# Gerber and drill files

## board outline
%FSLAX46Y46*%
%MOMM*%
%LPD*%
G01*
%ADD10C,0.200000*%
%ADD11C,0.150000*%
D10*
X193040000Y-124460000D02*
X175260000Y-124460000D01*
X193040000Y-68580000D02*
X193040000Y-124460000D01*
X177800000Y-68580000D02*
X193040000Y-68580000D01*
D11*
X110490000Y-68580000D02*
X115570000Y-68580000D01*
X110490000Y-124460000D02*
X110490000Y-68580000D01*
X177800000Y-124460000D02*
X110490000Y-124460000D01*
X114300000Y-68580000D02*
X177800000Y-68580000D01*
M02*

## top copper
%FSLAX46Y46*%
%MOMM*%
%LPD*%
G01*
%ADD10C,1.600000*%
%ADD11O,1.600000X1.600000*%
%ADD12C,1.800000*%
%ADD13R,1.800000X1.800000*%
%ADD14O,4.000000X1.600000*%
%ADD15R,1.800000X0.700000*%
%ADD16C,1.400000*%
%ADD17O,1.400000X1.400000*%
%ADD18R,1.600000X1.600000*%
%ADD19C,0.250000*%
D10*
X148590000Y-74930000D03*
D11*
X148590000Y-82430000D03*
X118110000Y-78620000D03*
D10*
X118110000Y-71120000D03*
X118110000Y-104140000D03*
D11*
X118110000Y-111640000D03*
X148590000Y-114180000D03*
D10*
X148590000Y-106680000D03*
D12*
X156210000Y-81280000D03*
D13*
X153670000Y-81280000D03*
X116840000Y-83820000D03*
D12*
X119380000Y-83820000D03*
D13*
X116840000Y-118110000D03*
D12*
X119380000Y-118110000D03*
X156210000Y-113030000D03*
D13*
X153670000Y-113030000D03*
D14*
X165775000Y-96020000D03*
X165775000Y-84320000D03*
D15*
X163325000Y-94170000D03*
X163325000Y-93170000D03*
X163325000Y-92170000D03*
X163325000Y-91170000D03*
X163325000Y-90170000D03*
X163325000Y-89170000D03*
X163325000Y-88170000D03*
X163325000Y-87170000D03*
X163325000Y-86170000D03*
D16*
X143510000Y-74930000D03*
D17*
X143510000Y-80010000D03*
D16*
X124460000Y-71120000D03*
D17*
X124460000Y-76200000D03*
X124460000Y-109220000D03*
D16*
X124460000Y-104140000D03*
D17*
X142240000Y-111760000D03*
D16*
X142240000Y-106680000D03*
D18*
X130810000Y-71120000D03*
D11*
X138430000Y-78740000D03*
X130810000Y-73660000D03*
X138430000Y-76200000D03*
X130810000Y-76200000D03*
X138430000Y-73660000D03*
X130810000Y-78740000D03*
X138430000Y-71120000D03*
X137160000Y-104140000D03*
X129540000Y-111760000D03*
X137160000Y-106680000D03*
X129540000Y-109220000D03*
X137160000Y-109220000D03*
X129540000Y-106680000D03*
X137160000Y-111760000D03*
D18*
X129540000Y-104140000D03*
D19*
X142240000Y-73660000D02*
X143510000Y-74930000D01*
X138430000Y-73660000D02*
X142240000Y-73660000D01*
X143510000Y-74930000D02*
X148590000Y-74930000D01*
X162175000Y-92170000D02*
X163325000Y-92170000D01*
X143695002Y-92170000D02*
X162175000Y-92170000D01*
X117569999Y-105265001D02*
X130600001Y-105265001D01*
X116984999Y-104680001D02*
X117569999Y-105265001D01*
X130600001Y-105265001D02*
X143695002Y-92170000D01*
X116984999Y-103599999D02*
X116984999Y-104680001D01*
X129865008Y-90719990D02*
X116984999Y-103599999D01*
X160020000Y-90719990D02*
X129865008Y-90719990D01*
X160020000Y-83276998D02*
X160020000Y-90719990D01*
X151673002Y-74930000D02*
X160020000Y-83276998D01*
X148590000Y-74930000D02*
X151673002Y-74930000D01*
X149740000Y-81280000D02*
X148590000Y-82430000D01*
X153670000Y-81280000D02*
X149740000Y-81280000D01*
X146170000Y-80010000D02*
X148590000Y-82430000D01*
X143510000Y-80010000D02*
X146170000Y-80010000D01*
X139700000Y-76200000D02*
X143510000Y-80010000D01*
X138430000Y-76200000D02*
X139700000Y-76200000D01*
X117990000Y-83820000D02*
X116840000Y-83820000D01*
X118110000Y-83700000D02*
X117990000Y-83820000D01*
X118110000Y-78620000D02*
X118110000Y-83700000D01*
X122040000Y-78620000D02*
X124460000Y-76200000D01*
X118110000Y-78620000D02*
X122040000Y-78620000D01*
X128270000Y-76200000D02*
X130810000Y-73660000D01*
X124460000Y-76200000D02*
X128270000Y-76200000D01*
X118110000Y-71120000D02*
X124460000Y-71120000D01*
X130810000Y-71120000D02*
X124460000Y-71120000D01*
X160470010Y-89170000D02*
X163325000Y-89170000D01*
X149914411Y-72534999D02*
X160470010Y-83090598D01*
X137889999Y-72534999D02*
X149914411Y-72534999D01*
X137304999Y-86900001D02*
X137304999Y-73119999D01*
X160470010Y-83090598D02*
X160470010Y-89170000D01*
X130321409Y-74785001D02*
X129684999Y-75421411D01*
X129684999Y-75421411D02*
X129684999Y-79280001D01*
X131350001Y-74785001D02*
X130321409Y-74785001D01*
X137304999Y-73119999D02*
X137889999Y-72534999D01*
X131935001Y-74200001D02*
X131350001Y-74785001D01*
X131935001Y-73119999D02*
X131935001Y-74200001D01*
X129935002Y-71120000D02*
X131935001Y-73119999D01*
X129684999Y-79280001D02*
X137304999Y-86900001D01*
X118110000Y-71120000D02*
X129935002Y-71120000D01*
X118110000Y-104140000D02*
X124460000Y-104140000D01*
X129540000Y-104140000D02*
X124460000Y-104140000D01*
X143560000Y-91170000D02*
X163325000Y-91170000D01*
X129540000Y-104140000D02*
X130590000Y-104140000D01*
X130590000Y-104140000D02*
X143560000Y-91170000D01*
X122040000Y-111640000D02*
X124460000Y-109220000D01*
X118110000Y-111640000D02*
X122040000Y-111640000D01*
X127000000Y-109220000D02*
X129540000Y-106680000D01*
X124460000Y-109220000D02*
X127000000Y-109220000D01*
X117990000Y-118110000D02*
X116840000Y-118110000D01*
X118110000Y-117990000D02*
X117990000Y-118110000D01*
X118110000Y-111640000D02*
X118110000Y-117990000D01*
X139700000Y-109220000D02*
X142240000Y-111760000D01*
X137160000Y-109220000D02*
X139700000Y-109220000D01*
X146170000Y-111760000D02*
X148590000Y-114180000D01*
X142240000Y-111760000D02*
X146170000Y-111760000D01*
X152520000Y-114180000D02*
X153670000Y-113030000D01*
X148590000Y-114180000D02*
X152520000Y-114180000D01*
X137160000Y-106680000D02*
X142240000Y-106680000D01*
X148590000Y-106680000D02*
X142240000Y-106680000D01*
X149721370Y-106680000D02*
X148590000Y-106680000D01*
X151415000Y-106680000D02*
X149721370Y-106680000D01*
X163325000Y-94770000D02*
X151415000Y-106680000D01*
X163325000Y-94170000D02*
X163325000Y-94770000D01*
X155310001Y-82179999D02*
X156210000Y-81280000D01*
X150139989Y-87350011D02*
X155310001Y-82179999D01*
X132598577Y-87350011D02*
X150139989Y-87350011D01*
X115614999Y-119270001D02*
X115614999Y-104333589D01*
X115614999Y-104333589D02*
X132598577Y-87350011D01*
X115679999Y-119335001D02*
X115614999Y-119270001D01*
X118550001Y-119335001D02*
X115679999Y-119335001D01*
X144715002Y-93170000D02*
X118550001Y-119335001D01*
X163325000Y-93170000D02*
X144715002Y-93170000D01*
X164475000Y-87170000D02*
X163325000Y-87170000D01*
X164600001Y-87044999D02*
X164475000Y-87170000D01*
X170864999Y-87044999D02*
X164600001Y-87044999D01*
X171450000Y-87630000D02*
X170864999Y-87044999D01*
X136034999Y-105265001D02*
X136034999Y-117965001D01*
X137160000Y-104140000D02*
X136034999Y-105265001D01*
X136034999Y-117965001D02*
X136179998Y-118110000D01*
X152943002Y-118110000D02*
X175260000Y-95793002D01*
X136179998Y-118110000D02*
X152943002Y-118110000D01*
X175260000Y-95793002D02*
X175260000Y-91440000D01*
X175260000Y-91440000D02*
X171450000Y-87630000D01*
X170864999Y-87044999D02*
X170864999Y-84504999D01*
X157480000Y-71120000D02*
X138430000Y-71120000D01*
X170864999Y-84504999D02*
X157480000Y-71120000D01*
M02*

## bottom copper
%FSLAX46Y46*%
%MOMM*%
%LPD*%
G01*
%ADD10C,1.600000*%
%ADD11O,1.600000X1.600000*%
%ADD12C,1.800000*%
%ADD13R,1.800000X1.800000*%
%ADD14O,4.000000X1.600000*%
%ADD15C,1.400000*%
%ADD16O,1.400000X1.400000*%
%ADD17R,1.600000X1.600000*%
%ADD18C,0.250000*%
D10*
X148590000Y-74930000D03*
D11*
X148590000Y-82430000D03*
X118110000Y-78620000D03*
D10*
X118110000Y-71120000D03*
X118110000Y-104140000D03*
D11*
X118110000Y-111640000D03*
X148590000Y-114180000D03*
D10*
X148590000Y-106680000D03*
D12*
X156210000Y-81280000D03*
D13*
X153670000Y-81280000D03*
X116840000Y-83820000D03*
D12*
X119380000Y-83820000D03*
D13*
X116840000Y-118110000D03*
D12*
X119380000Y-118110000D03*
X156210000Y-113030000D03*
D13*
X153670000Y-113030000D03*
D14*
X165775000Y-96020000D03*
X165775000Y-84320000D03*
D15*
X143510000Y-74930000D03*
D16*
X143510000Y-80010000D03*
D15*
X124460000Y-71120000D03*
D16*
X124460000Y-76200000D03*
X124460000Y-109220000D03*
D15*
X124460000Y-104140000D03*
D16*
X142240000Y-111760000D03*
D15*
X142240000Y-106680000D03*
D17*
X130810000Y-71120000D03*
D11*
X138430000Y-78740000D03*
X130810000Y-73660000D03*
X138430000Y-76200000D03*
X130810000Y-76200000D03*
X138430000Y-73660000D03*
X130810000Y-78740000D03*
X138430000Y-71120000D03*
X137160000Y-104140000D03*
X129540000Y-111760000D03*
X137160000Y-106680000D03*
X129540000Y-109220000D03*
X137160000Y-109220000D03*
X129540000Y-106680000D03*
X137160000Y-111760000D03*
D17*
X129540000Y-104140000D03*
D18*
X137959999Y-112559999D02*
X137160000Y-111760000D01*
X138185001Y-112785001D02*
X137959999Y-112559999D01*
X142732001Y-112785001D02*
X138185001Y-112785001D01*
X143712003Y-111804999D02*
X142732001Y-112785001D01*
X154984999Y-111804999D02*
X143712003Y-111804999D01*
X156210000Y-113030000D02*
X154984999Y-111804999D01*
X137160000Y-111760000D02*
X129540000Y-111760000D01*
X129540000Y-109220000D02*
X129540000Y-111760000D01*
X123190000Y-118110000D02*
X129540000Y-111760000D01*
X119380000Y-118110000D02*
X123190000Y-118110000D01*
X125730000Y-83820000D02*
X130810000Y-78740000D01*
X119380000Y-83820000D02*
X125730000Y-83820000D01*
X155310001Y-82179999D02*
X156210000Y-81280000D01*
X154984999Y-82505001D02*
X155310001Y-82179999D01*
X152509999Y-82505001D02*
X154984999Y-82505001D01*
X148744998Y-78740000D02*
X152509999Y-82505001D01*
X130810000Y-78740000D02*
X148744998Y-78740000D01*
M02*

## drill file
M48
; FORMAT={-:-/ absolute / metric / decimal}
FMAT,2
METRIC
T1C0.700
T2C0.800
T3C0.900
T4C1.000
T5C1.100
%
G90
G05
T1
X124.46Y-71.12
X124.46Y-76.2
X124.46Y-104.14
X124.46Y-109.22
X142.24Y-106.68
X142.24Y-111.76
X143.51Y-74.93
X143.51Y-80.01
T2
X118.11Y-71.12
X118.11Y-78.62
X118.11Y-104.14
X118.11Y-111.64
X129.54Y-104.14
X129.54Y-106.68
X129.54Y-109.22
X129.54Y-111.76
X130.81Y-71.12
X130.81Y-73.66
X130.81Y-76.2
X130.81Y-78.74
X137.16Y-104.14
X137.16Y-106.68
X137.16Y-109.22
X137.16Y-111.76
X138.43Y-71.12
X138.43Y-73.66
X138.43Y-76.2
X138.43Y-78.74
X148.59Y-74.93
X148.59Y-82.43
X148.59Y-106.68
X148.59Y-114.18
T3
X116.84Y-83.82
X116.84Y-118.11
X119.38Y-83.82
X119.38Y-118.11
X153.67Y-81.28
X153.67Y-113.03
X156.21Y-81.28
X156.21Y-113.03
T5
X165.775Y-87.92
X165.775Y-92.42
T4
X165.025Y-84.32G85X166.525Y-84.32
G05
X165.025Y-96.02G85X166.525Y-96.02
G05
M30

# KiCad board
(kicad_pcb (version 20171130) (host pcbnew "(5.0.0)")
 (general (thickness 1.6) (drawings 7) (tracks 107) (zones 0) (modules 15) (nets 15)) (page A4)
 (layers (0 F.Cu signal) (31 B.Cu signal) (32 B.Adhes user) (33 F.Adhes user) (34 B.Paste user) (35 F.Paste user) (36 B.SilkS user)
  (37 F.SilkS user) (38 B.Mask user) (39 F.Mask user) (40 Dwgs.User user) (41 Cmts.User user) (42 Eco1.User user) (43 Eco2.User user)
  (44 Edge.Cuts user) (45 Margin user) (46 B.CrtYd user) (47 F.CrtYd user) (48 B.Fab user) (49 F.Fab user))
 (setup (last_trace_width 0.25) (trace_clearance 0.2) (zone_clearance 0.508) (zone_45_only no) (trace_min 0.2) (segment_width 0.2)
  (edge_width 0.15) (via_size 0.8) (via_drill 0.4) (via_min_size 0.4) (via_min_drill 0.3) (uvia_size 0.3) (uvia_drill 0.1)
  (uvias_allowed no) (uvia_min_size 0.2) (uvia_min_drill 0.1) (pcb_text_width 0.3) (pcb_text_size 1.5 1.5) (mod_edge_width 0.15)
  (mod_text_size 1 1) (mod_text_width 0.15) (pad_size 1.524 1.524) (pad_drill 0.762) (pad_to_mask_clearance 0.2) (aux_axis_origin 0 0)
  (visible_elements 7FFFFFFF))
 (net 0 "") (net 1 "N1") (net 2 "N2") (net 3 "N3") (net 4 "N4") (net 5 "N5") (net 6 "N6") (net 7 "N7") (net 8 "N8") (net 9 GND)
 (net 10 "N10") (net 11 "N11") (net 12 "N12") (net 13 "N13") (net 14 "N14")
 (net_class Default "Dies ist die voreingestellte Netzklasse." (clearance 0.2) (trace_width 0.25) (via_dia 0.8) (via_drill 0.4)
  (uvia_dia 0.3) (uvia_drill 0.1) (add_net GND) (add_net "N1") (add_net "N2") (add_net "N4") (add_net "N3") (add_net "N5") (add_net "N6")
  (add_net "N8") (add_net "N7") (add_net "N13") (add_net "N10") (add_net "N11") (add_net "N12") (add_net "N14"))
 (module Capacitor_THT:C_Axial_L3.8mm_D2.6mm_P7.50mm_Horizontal (layer F.Cu) (at 148.59 74.93 270)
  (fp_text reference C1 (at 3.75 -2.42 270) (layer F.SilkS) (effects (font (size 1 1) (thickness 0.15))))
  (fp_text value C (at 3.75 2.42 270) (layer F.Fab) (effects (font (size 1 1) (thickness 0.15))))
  (pad 1 thru_hole circle (at 0 0 270) (size 1.6 1.6) (drill 0.8) (layers *.Cu *.Mask) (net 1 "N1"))
  (pad 2 thru_hole oval (at 7.5 0 270) (size 1.6 1.6) (drill 0.8) (layers *.Cu *.Mask) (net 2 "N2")))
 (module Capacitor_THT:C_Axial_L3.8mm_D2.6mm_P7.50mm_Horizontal (layer F.Cu) (at 118.11 71.12 270)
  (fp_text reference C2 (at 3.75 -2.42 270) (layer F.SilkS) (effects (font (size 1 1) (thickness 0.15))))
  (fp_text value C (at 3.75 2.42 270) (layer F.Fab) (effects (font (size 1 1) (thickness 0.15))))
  (pad 2 thru_hole oval (at 7.5 0 270) (size 1.6 1.6) (drill 0.8) (layers *.Cu *.Mask) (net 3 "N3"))
  (pad 1 thru_hole circle (at 0 0 270) (size 1.6 1.6) (drill 0.8) (layers *.Cu *.Mask) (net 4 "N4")))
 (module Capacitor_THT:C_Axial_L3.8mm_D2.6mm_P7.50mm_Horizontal (layer F.Cu) (at 118.11 104.14 270)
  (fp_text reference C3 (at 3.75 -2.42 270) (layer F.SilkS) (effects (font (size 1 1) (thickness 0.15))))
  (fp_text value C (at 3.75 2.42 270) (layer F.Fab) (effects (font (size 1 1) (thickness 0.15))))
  (pad 1 thru_hole circle (at 0 0 270) (size 1.6 1.6) (drill 0.8) (layers *.Cu *.Mask) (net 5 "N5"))
  (pad 2 thru_hole oval (at 7.5 0 270) (size 1.6 1.6) (drill 0.8) (layers *.Cu *.Mask) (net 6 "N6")))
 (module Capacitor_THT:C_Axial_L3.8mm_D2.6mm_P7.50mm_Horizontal (layer F.Cu) (at 148.59 106.68 270)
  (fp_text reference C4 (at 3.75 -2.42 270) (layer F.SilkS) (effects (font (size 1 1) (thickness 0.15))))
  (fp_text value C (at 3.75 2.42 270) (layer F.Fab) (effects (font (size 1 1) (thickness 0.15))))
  (pad 2 thru_hole oval (at 7.5 0 270) (size 1.6 1.6) (drill 0.8) (layers *.Cu *.Mask) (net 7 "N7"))
  (pad 1 thru_hole circle (at 0 0 270) (size 1.6 1.6) (drill 0.8) (layers *.Cu *.Mask) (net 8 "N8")))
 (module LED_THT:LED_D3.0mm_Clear (layer F.Cu) (at 153.67 81.28)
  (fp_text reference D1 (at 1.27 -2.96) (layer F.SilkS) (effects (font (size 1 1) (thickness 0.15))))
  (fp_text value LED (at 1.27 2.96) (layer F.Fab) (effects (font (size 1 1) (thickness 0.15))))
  (pad 2 thru_hole circle (at 2.54 0) (size 1.8 1.8) (drill 0.9) (layers *.Cu *.Mask) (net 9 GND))
  (pad 1 thru_hole rect (at 0 0) (size 1.8 1.8) (drill 0.9) (layers *.Cu *.Mask) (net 2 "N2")))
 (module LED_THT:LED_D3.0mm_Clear (layer F.Cu) (at 116.84 83.82)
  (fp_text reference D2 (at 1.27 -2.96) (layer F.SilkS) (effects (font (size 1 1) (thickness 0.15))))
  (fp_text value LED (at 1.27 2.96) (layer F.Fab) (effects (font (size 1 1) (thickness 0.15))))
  (pad 1 thru_hole rect (at 0 0) (size 1.8 1.8) (drill 0.9) (layers *.Cu *.Mask) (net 3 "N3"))
  (pad 2 thru_hole circle (at 2.54 0) (size 1.8 1.8) (drill 0.9) (layers *.Cu *.Mask) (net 9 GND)))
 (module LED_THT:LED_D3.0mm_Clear (layer F.Cu) (at 116.84 118.11)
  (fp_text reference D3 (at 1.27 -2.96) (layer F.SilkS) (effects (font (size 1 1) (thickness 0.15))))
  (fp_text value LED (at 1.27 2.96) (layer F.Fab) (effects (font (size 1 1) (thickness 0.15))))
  (pad 1 thru_hole rect (at 0 0) (size 1.8 1.8) (drill 0.9) (layers *.Cu *.Mask) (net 6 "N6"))
  (pad 2 thru_hole circle (at 2.54 0) (size 1.8 1.8) (drill 0.9) (layers *.Cu *.Mask) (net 9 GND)))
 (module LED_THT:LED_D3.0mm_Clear (layer F.Cu) (at 153.67 113.03)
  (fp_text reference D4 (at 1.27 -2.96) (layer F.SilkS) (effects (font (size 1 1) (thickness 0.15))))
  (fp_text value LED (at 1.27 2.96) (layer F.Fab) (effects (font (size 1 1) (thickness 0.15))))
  (pad 2 thru_hole circle (at 2.54 0) (size 1.8 1.8) (drill 0.9) (layers *.Cu *.Mask) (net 9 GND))
  (pad 1 thru_hole rect (at 0 0) (size 1.8 1.8) (drill 0.9) (layers *.Cu *.Mask) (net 7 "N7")))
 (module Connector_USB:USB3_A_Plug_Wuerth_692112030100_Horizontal (layer F.Cu) (at 165.1 90.17)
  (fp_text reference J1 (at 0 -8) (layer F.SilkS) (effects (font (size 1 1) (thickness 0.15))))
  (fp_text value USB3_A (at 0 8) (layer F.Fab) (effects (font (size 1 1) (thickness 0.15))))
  (pad 10 thru_hole oval (at 0.675 5.85 90) (size 1.6 4) (drill oval 1 2.5) (layers *.Cu *.Mask) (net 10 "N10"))
  (pad 10 thru_hole oval (at 0.675 -5.85 90) (size 1.6 4) (drill oval 1 2.5) (layers *.Cu *.Mask) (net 10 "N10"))
  (pad 5 smd rect (at -1.775 4 90) (size 0.7 1.8) (layers F.Cu F.Paste F.Mask) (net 8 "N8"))
  (pad 4 smd rect (at -1.775 3 90) (size 0.7 1.8) (layers F.Cu F.Paste F.Mask) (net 9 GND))
  (pad 6 smd rect (at -1.775 2 90) (size 0.7 1.8) (layers F.Cu F.Paste F.Mask) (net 1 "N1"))
  (pad 3 smd rect (at -1.775 1 90) (size 0.7 1.8) (layers F.Cu F.Paste F.Mask) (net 5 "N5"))
  (pad 7 smd rect (at -1.775 0 90) (size 0.7 1.8) (layers F.Cu F.Paste F.Mask) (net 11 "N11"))
  (pad 2 smd rect (at -1.775 -1 90) (size 0.7 1.8) (layers F.Cu F.Paste F.Mask) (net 4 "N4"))
  (pad 8 smd rect (at -1.775 -2 90) (size 0.7 1.8) (layers F.Cu F.Paste F.Mask) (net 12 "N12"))
  (pad 1 smd rect (at -1.775 -3 90) (size 0.7 1.8) (layers F.Cu F.Paste F.Mask) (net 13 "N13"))
  (pad 9 smd rect (at -1.775 -4) (size 1.8 0.7) (layers F.Cu F.Paste F.Mask) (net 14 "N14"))
  (pad "" np_thru_hole circle (at 0.675 2.25 90) (size 1.1 1.1) (drill 1.1) (layers *.Cu *.Mask))
  (pad "" np_thru_hole circle (at 0.675 -2.25 90) (size 1.1 1.1) (drill 1.1) (layers *.Cu *.Mask)))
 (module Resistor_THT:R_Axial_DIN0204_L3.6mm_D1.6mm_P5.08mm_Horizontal (layer F.Cu) (at 143.51 74.93 270)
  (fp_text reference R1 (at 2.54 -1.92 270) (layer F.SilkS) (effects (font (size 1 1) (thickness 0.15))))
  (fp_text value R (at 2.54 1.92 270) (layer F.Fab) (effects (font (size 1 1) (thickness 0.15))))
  (pad 1 thru_hole circle (at 0 0 270) (size 1.4 1.4) (drill 0.7) (layers *.Cu *.Mask) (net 1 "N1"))
  (pad 2 thru_hole oval (at 5.08 0 270) (size 1.4 1.4) (drill 0.7) (layers *.Cu *.Mask) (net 2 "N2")))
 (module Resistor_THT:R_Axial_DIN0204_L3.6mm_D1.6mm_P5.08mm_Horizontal (layer F.Cu) (at 124.46 71.12 270)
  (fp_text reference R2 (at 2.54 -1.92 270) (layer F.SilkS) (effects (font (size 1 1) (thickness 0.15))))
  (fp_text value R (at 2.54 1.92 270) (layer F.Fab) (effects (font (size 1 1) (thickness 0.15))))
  (pad 1 thru_hole circle (at 0 0 270) (size 1.4 1.4) (drill 0.7) (layers *.Cu *.Mask) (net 4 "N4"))
  (pad 2 thru_hole oval (at 5.08 0 270) (size 1.4 1.4) (drill 0.7) (layers *.Cu *.Mask) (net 3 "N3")))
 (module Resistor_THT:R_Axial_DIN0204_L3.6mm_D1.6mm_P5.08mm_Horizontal (layer F.Cu) (at 124.46 104.14 270)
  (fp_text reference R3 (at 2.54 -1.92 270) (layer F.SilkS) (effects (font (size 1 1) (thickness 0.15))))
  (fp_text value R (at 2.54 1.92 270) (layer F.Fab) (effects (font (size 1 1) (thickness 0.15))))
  (pad 2 thru_hole oval (at 5.08 0 270) (size 1.4 1.4) (drill 0.7) (layers *.Cu *.Mask) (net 6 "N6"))
  (pad 1 thru_hole circle (at 0 0 270) (size 1.4 1.4) (drill 0.7) (layers *.Cu *.Mask) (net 5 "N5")))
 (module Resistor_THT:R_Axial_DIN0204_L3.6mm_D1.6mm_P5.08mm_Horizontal (layer F.Cu) (at 142.24 106.68 270)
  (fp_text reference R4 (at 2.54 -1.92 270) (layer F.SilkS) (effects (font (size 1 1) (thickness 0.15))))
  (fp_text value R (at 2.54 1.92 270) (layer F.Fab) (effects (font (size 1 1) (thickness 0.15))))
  (pad 2 thru_hole oval (at 5.08 0 270) (size 1.4 1.4) (drill 0.7) (layers *.Cu *.Mask) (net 7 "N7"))
  (pad 1 thru_hole circle (at 0 0 270) (size 1.4 1.4) (drill 0.7) (layers *.Cu *.Mask) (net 8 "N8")))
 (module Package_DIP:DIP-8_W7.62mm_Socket (layer F.Cu) (at 130.81 71.12)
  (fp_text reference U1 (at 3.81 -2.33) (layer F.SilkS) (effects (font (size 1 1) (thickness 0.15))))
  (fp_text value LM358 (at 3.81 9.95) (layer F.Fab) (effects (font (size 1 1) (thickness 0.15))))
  (pad 1 thru_hole rect (at 0 0) (size 1.6 1.6) (drill 0.8) (layers *.Cu *.Mask) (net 4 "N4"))
  (pad 5 thru_hole oval (at 7.62 7.62) (size 1.6 1.6) (drill 0.8) (layers *.Cu *.Mask) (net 9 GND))
  (pad 2 thru_hole oval (at 0 2.54) (size 1.6 1.6) (drill 0.8) (layers *.Cu *.Mask) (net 3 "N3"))
  (pad 6 thru_hole oval (at 7.62 5.08) (size 1.6 1.6) (drill 0.8) (layers *.Cu *.Mask) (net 2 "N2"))
  (pad 3 thru_hole oval (at 0 5.08) (size 1.6 1.6) (drill 0.8) (layers *.Cu *.Mask) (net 9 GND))
  (pad 7 thru_hole oval (at 7.62 2.54) (size 1.6 1.6) (drill 0.8) (layers *.Cu *.Mask) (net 1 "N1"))
  (pad 4 thru_hole oval (at 0 7.62) (size 1.6 1.6) (drill 0.8) (layers *.Cu *.Mask) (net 9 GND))
  (pad 8 thru_hole oval (at 7.62 0) (size 1.6 1.6) (drill 0.8) (layers *.Cu *.Mask) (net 13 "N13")))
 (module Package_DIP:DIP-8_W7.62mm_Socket (layer F.Cu) (at 129.54 104.14)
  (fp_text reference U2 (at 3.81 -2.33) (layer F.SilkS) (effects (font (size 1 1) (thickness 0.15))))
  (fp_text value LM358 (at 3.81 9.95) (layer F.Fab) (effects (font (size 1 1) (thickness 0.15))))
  (pad 8 thru_hole oval (at 7.62 0) (size 1.6 1.6) (drill 0.8) (layers *.Cu *.Mask) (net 13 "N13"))
  (pad 4 thru_hole oval (at 0 7.62) (size 1.6 1.6) (drill 0.8) (layers *.Cu *.Mask) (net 9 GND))
  (pad 7 thru_hole oval (at 7.62 2.54) (size 1.6 1.6) (drill 0.8) (layers *.Cu *.Mask) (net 8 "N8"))
  (pad 3 thru_hole oval (at 0 5.08) (size 1.6 1.6) (drill 0.8) (layers *.Cu *.Mask) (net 9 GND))
  (pad 6 thru_hole oval (at 7.62 5.08) (size 1.6 1.6) (drill 0.8) (layers *.Cu *.Mask) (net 7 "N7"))
  (pad 2 thru_hole oval (at 0 2.54) (size 1.6 1.6) (drill 0.8) (layers *.Cu *.Mask) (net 6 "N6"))
  (pad 5 thru_hole oval (at 7.62 7.62) (size 1.6 1.6) (drill 0.8) (layers *.Cu *.Mask) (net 9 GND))
  (pad 1 thru_hole rect (at 0 0) (size 1.6 1.6) (drill 0.8) (layers *.Cu *.Mask) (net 5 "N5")))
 (gr_line (start 193.04 124.46) (end 175.26 124.46) (layer Edge.Cuts) (width 0.2))
 (gr_line (start 193.04 68.58) (end 193.04 124.46) (layer Edge.Cuts) (width 0.2))
 (gr_line (start 177.8 68.58) (end 193.04 68.58) (layer Edge.Cuts) (width 0.2))
 (gr_line (start 110.49 68.58) (end 115.57 68.58) (layer Edge.Cuts) (width 0.15))
 (gr_line (start 110.49 124.46) (end 110.49 68.58) (layer Edge.Cuts) (width 0.15))
 (gr_line (start 177.8 124.46) (end 110.49 124.46) (layer Edge.Cuts) (width 0.15))
 (gr_line (start 114.3 68.58) (end 177.8 68.58) (layer Edge.Cuts) (width 0.15))
 (segment (start 142.24 73.66) (end 143.51 74.93) (width 0.25) (layer F.Cu) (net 1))
 (segment (start 138.43 73.66) (end 142.24 73.66) (width 0.25) (layer F.Cu) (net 1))
 (segment (start 143.51 74.93) (end 148.59 74.93) (width 0.25) (layer F.Cu) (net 1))
 (segment (start 162.175 92.17) (end 163.325 92.17) (width 0.25) (layer F.Cu) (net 1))
 (segment (start 143.695002 92.17) (end 162.175 92.17) (width 0.25) (layer F.Cu) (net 1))
 (segment (start 117.569999 105.265001) (end 130.600001 105.265001) (width 0.25) (layer F.Cu) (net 1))
 (segment (start 116.984999 104.680001) (end 117.569999 105.265001) (width 0.25) (layer F.Cu) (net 1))
 (segment (start 130.600001 105.265001) (end 143.695002 92.17) (width 0.25) (layer F.Cu) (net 1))
 (segment (start 116.984999 103.599999) (end 116.984999 104.680001) (width 0.25) (layer F.Cu) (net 1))
 (segment (start 129.865008 90.71999) (end 116.984999 103.599999) (width 0.25) (layer F.Cu) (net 1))
 (segment (start 160.02 90.71999) (end 129.865008 90.71999) (width 0.25) (layer F.Cu) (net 1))
 (segment (start 160.02 83.276998) (end 160.02 90.71999) (width 0.25) (layer F.Cu) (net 1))
 (segment (start 151.673002 74.93) (end 160.02 83.276998) (width 0.25) (layer F.Cu) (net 1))
 (segment (start 148.59 74.93) (end 151.673002 74.93) (width 0.25) (layer F.Cu) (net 1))
 (segment (start 149.74 81.28) (end 148.59 82.43) (width 0.25) (layer F.Cu) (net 2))
 (segment (start 153.67 81.28) (end 149.74 81.28) (width 0.25) (layer F.Cu) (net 2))
 (segment (start 146.17 80.01) (end 148.59 82.43) (width 0.25) (layer F.Cu) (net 2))
 (segment (start 143.51 80.01) (end 146.17 80.01) (width 0.25) (layer F.Cu) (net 2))
 (segment (start 139.7 76.2) (end 143.51 80.01) (width 0.25) (layer F.Cu) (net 2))
 (segment (start 138.43 76.2) (end 139.7 76.2) (width 0.25) (layer F.Cu) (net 2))
 (segment (start 117.99 83.82) (end 116.84 83.82) (width 0.25) (layer F.Cu) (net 3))
 (segment (start 118.11 83.7) (end 117.99 83.82) (width 0.25) (layer F.Cu) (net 3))
 (segment (start 118.11 78.62) (end 118.11 83.7) (width 0.25) (layer F.Cu) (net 3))
 (segment (start 122.04 78.62) (end 124.46 76.2) (width 0.25) (layer F.Cu) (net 3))
 (segment (start 118.11 78.62) (end 122.04 78.62) (width 0.25) (layer F.Cu) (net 3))
 (segment (start 128.27 76.2) (end 130.81 73.66) (width 0.25) (layer F.Cu) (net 3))
 (segment (start 124.46 76.2) (end 128.27 76.2) (width 0.25) (layer F.Cu) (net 3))
 (segment (start 118.11 71.12) (end 124.46 71.12) (width 0.25) (layer F.Cu) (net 4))
 (segment (start 130.81 71.12) (end 124.46 71.12) (width 0.25) (layer F.Cu) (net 4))
 (segment (start 160.47001 89.17) (end 163.325 89.17) (width 0.25) (layer F.Cu) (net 4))
 (segment (start 149.914411 72.534999) (end 160.47001 83.090598) (width 0.25) (layer F.Cu) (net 4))
 (segment (start 137.889999 72.534999) (end 149.914411 72.534999) (width 0.25) (layer F.Cu) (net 4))
 (segment (start 137.304999 86.900001) (end 137.304999 73.119999) (width 0.25) (layer F.Cu) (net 4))
 (segment (start 160.47001 83.090598) (end 160.47001 89.17) (width 0.25) (layer F.Cu) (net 4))
 (segment (start 130.321409 74.785001) (end 129.684999 75.421411) (width 0.25) (layer F.Cu) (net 4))
 (segment (start 129.684999 75.421411) (end 129.684999 79.280001) (width 0.25) (layer F.Cu) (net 4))
 (segment (start 131.350001 74.785001) (end 130.321409 74.785001) (width 0.25) (layer F.Cu) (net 4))
 (segment (start 137.304999 73.119999) (end 137.889999 72.534999) (width 0.25) (layer F.Cu) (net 4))
 (segment (start 131.935001 74.200001) (end 131.350001 74.785001) (width 0.25) (layer F.Cu) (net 4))
 (segment (start 131.935001 73.119999) (end 131.935001 74.200001) (width 0.25) (layer F.Cu) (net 4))
 (segment (start 129.935002 71.12) (end 131.935001 73.119999) (width 0.25) (layer F.Cu) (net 4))
 (segment (start 129.684999 79.280001) (end 137.304999 86.900001) (width 0.25) (layer F.Cu) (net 4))
 (segment (start 118.11 71.12) (end 129.935002 71.12) (width 0.25) (layer F.Cu) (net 4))
 (segment (start 118.11 104.14) (end 124.46 104.14) (width 0.25) (layer F.Cu) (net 5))
 (segment (start 129.54 104.14) (end 124.46 104.14) (width 0.25) (layer F.Cu) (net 5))
 (segment (start 143.56 91.17) (end 163.325 91.17) (width 0.25) (layer F.Cu) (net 5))
 (segment (start 129.54 104.14) (end 130.59 104.14) (width 0.25) (layer F.Cu) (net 5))
 (segment (start 130.59 104.14) (end 143.56 91.17) (width 0.25) (layer F.Cu) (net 5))
 (segment (start 122.04 111.64) (end 124.46 109.22) (width 0.25) (layer F.Cu) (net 6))
 (segment (start 118.11 111.64) (end 122.04 111.64) (width 0.25) (layer F.Cu) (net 6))
 (segment (start 127 109.22) (end 129.54 106.68) (width 0.25) (layer F.Cu) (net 6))
 (segment (start 124.46 109.22) (end 127 109.22) (width 0.25) (layer F.Cu) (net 6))
 (segment (start 117.99 118.11) (end 116.84 118.11) (width 0.25) (layer F.Cu) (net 6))
 (segment (start 118.11 117.99) (end 117.99 118.11) (width 0.25) (layer F.Cu) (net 6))
 (segment (start 118.11 111.64) (end 118.11 117.99) (width 0.25) (layer F.Cu) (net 6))
 (segment (start 139.7 109.22) (end 142.24 111.76) (width 0.25) (layer F.Cu) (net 7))
 (segment (start 137.16 109.22) (end 139.7 109.22) (width 0.25) (layer F.Cu) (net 7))
 (segment (start 146.17 111.76) (end 148.59 114.18) (width 0.25) (layer F.Cu) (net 7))
 (segment (start 142.24 111.76) (end 146.17 111.76) (width 0.25) (layer F.Cu) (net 7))
 (segment (start 152.52 114.18) (end 153.67 113.03) (width 0.25) (layer F.Cu) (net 7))
 (segment (start 148.59 114.18) (end 152.52 114.18) (width 0.25) (layer F.Cu) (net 7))
 (segment (start 137.16 106.68) (end 142.24 106.68) (width 0.25) (layer F.Cu) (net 8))
 (segment (start 148.59 106.68) (end 142.24 106.68) (width 0.25) (layer F.Cu) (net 8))
 (segment (start 149.72137 106.68) (end 148.59 106.68) (width 0.25) (layer F.Cu) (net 8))
 (segment (start 151.415 106.68) (end 149.72137 106.68) (width 0.25) (layer F.Cu) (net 8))
 (segment (start 163.325 94.77) (end 151.415 106.68) (width 0.25) (layer F.Cu) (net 8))
 (segment (start 163.325 94.17) (end 163.325 94.77) (width 0.25) (layer F.Cu) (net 8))
 (segment (start 137.959999 112.559999) (end 137.16 111.76) (width 0.25) (layer B.Cu) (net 9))
 (segment (start 138.185001 112.785001) (end 137.959999 112.559999) (width 0.25) (layer B.Cu) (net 9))
 (segment (start 142.732001 112.785001) (end 138.185001 112.785001) (width 0.25) (layer B.Cu) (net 9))
 (segment (start 143.712003 111.804999) (end 142.732001 112.785001) (width 0.25) (layer B.Cu) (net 9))
 (segment (start 154.984999 111.804999) (end 143.712003 111.804999) (width 0.25) (layer B.Cu) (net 9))
 (segment (start 156.21 113.03) (end 154.984999 111.804999) (width 0.25) (layer B.Cu) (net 9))
 (segment (start 137.16 111.76) (end 129.54 111.76) (width 0.25) (layer B.Cu) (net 9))
 (segment (start 129.54 109.22) (end 129.54 111.76) (width 0.25) (layer B.Cu) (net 9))
 (segment (start 123.19 118.11) (end 129.54 111.76) (width 0.25) (layer B.Cu) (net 9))
 (segment (start 119.38 118.11) (end 123.19 118.11) (width 0.25) (layer B.Cu) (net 9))
 (segment (start 125.73 83.82) (end 130.81 78.74) (width 0.25) (layer B.Cu) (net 9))
 (segment (start 119.38 83.82) (end 125.73 83.82) (width 0.25) (layer B.Cu) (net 9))
 (segment (start 155.310001 82.179999) (end 156.21 81.28) (width 0.25) (layer B.Cu) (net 9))
 (segment (start 154.984999 82.505001) (end 155.310001 82.179999) (width 0.25) (layer B.Cu) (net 9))
 (segment (start 152.509999 82.505001) (end 154.984999 82.505001) (width 0.25) (layer B.Cu) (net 9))
 (segment (start 148.744998 78.74) (end 152.509999 82.505001) (width 0.25) (layer B.Cu) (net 9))
 (segment (start 130.81 78.74) (end 148.744998 78.74) (width 0.25) (layer B.Cu) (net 9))
 (segment (start 155.310001 82.179999) (end 156.21 81.28) (width 0.25) (layer F.Cu) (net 9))
 (segment (start 150.139989 87.350011) (end 155.310001 82.179999) (width 0.25) (layer F.Cu) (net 9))
 (segment (start 132.598577 87.350011) (end 150.139989 87.350011) (width 0.25) (layer F.Cu) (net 9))
 (segment (start 115.614999 119.270001) (end 115.614999 104.333589) (width 0.25) (layer F.Cu) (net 9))
 (segment (start 115.614999 104.333589) (end 132.598577 87.350011) (width 0.25) (layer F.Cu) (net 9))
 (segment (start 115.679999 119.335001) (end 115.614999 119.270001) (width 0.25) (layer F.Cu) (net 9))
 (segment (start 118.550001 119.335001) (end 115.679999 119.335001) (width 0.25) (layer F.Cu) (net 9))
 (segment (start 144.715002 93.17) (end 118.550001 119.335001) (width 0.25) (layer F.Cu) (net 9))
 (segment (start 163.325 93.17) (end 144.715002 93.17) (width 0.25) (layer F.Cu) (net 9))
 (segment (start 164.475 87.17) (end 163.325 87.17) (width 0.25) (layer F.Cu) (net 13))
 (segment (start 164.600001 87.044999) (end 164.475 87.17) (width 0.25) (layer F.Cu) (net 13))
 (segment (start 170.864999 87.044999) (end 164.600001 87.044999) (width 0.25) (layer F.Cu) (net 13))
 (segment (start 171.45 87.63) (end 170.864999 87.044999) (width 0.25) (layer F.Cu) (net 13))
 (segment (start 136.034999 105.265001) (end 136.034999 117.965001) (width 0.25) (layer F.Cu) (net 13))
 (segment (start 137.16 104.14) (end 136.034999 105.265001) (width 0.25) (layer F.Cu) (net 13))
 (segment (start 136.034999 117.965001) (end 136.179998 118.11) (width 0.25) (layer F.Cu) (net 13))
 (segment (start 152.943002 118.11) (end 175.26 95.793002) (width 0.25) (layer F.Cu) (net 13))
 (segment (start 136.179998 118.11) (end 152.943002 118.11) (width 0.25) (layer F.Cu) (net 13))
 (segment (start 175.26 95.793002) (end 175.26 91.44) (width 0.25) (layer F.Cu) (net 13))
 (segment (start 175.26 91.44) (end 171.45 87.63) (width 0.25) (layer F.Cu) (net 13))
 (segment (start 170.864999 87.044999) (end 170.864999 84.504999) (width 0.25) (layer F.Cu) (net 13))
 (segment (start 157.48 71.12) (end 138.43 71.12) (width 0.25) (layer F.Cu) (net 13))
 (segment (start 170.864999 84.504999) (end 157.48 71.12) (width 0.25) (layer F.Cu) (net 13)))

